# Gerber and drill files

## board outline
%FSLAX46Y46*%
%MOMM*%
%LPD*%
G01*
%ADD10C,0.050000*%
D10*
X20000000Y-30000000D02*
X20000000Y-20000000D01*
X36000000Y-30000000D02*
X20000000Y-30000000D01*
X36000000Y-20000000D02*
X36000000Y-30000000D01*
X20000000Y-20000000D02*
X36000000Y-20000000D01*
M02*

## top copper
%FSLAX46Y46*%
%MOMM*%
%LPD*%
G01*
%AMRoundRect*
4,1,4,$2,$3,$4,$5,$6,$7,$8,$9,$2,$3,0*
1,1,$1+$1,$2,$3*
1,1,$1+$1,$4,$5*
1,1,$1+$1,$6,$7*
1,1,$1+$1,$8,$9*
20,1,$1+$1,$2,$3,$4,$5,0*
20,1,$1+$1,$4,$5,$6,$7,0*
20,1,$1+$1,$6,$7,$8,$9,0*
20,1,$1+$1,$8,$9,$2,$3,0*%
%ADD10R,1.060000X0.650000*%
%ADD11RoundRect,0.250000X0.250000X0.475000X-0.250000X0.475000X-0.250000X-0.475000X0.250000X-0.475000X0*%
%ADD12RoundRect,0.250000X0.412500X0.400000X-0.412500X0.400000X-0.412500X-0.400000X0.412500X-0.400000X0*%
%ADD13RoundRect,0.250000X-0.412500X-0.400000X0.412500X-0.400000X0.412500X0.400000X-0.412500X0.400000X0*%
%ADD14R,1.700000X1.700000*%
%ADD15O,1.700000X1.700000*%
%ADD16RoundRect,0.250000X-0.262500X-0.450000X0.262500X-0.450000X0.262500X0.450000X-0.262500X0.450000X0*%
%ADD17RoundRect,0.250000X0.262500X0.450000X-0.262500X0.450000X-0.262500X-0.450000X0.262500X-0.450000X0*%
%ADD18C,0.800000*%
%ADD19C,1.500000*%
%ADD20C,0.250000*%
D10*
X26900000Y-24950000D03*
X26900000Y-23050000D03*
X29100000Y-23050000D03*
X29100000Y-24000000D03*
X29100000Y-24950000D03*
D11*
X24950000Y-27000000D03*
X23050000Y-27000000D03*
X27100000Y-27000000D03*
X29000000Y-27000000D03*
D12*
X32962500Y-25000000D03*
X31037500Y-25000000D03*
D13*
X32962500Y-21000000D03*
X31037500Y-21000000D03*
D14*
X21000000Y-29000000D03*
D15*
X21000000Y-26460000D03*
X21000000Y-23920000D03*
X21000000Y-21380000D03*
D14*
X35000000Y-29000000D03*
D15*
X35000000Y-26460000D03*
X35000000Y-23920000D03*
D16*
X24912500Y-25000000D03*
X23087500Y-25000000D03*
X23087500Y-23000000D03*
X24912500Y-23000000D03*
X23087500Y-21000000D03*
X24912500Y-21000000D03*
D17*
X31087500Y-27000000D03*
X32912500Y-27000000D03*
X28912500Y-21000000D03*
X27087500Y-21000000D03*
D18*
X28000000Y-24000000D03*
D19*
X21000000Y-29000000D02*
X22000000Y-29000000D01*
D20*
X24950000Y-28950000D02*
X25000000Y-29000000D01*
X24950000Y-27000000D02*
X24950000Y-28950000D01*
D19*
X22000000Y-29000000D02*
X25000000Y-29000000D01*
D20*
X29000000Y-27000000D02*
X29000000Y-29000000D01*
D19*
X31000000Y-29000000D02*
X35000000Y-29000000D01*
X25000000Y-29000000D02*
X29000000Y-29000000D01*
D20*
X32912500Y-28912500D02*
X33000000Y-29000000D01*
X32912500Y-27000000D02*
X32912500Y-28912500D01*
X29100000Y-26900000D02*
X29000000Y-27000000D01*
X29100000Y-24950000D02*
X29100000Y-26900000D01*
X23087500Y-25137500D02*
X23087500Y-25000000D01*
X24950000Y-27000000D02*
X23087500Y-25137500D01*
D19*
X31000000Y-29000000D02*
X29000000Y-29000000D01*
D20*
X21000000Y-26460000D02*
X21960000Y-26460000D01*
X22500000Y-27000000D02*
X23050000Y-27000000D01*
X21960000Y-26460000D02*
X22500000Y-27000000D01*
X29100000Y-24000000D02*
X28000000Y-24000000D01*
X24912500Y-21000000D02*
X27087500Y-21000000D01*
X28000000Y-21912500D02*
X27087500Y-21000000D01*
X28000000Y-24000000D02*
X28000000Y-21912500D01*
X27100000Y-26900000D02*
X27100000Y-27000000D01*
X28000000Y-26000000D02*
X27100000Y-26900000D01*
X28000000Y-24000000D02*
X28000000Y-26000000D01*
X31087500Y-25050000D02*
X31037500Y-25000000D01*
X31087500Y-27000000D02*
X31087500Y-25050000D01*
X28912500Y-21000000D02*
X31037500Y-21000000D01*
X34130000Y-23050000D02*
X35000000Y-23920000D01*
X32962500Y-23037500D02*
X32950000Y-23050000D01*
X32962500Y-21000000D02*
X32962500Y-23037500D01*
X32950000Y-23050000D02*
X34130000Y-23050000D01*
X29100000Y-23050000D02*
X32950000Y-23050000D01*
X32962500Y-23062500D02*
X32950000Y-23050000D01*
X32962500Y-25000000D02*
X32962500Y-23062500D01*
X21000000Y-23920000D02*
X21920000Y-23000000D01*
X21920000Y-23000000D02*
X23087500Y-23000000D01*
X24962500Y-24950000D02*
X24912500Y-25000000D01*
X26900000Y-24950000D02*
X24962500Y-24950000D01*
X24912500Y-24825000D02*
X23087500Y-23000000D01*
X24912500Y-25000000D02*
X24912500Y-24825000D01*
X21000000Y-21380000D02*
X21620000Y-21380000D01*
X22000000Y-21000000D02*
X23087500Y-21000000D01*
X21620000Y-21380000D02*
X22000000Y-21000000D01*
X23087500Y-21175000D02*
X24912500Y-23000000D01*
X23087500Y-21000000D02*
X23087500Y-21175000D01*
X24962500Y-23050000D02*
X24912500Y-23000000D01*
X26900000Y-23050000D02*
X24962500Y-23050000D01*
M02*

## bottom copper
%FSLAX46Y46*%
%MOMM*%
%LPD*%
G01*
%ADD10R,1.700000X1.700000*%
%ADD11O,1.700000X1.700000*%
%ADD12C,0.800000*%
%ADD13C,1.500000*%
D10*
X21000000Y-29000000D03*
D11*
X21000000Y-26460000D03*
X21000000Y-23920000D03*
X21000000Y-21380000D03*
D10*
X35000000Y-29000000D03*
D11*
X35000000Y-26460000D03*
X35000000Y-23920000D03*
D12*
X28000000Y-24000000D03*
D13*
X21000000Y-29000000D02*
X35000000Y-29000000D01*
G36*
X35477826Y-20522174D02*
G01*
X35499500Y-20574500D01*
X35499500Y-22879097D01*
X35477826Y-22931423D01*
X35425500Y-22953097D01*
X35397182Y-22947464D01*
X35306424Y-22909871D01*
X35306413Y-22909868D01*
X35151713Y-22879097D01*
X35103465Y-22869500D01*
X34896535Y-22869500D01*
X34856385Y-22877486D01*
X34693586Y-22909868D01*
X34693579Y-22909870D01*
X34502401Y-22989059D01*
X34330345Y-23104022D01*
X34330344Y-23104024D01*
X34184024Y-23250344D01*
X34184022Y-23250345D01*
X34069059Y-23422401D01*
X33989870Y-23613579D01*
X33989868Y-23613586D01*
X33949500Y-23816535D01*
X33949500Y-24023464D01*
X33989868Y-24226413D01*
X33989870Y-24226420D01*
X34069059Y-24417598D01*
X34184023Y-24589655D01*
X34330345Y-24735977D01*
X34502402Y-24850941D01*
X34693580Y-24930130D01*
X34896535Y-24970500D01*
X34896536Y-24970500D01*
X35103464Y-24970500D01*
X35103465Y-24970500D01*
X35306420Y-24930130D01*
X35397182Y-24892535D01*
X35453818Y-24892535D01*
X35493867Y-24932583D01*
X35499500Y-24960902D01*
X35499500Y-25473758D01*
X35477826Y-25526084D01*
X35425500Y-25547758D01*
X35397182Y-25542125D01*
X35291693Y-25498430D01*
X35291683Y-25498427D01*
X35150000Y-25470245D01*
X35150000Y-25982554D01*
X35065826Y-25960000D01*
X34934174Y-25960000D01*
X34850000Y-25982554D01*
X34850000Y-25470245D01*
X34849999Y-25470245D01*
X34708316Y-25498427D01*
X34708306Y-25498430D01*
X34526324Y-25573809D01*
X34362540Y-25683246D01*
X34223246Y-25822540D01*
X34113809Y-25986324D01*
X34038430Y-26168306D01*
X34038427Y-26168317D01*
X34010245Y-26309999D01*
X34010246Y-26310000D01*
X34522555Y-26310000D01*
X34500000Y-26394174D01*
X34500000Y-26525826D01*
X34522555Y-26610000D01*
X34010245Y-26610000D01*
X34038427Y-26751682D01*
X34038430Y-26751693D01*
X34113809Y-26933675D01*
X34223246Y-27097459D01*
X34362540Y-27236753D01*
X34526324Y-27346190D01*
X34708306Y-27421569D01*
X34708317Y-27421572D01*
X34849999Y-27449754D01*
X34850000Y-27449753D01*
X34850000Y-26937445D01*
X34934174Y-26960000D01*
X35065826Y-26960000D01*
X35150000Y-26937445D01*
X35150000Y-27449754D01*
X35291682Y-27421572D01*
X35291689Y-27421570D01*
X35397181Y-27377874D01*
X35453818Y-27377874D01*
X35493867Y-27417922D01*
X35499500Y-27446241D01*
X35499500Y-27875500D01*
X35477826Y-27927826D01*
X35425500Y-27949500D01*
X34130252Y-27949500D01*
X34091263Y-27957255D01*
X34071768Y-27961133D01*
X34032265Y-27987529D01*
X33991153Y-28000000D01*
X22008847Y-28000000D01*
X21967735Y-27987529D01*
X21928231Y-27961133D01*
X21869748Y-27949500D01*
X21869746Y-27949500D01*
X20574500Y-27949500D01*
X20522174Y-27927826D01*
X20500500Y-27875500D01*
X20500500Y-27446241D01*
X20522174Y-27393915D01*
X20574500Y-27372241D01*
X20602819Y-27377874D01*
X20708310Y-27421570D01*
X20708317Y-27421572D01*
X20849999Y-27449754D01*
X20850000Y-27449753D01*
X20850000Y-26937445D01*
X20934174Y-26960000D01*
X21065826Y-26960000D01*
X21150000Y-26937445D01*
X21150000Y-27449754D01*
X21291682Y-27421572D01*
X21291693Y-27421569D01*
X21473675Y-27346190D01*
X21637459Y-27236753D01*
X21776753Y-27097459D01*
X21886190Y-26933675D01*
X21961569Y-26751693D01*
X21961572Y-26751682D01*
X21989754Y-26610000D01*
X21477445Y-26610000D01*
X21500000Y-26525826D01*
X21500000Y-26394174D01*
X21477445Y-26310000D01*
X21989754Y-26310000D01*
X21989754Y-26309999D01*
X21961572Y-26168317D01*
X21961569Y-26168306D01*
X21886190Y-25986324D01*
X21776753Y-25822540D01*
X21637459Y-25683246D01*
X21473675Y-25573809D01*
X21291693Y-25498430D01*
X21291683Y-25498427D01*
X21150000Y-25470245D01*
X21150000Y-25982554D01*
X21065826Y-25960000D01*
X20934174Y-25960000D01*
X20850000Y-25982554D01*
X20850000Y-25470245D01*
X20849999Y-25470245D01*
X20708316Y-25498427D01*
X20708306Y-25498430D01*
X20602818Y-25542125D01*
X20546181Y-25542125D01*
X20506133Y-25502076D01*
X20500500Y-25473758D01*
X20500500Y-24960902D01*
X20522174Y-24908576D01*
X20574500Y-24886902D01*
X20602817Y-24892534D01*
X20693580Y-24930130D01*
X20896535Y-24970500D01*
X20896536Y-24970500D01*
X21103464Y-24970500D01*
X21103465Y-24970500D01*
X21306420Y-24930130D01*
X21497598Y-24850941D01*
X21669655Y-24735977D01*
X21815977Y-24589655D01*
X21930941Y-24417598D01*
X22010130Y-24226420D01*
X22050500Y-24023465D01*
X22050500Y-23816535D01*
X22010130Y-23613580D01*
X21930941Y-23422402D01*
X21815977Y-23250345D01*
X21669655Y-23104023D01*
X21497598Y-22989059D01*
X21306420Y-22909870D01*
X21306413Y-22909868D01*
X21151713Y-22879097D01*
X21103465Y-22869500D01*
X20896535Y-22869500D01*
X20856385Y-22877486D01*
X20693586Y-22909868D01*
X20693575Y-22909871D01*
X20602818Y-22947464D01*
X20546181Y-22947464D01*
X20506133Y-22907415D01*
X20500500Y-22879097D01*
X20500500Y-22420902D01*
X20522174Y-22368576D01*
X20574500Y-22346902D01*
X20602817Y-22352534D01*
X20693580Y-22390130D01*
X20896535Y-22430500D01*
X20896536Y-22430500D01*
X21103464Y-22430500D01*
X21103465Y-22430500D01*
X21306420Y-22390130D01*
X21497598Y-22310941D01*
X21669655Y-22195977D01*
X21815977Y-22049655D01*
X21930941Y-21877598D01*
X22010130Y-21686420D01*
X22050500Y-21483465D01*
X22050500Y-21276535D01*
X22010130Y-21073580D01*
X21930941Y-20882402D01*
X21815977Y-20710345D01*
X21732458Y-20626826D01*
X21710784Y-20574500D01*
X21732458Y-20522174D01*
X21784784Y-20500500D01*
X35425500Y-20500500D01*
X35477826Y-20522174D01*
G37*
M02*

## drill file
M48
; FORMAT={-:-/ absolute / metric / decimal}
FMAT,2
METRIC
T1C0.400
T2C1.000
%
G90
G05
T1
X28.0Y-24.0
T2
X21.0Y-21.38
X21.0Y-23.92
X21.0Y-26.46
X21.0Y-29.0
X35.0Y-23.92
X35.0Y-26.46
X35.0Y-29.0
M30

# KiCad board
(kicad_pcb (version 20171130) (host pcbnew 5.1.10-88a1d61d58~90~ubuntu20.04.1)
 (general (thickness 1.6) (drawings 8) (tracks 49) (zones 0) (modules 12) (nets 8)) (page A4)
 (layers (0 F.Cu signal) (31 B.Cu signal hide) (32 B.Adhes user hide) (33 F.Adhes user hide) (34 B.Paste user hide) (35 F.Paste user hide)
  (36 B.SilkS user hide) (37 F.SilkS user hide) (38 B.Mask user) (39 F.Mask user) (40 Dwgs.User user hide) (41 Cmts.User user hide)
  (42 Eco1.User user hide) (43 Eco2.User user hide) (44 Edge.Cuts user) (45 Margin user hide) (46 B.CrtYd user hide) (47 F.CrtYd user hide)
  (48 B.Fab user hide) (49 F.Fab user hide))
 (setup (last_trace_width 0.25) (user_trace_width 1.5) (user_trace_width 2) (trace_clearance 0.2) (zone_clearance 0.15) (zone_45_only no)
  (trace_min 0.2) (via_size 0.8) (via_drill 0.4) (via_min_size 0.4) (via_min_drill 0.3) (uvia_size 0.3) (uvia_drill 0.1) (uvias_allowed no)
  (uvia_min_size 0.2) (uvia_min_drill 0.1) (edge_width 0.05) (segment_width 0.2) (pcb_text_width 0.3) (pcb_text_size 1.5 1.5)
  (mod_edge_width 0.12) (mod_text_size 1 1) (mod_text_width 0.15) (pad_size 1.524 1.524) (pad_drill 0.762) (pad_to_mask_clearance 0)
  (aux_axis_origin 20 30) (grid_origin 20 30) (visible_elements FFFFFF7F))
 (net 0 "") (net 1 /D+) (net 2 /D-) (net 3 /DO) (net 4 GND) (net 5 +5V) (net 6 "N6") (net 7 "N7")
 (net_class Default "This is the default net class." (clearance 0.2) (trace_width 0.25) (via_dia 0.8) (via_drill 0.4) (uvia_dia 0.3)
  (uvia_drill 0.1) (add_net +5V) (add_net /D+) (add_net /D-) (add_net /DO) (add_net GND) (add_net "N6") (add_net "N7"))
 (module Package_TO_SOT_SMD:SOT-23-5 (layer F.Cu) (at 28 24 180)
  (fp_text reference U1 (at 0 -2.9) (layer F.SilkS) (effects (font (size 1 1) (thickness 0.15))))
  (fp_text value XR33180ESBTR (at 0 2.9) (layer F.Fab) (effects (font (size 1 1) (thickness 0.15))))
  (pad 5 smd rect (at 1.1 -0.95 180) (size 1.06 0.65) (layers F.Cu F.Paste F.Mask) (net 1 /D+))
  (pad 4 smd rect (at 1.1 0.95 180) (size 1.06 0.65) (layers F.Cu F.Paste F.Mask) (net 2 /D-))
  (pad 3 smd rect (at -1.1 0.95 180) (size 1.06 0.65) (layers F.Cu F.Paste F.Mask) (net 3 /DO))
  (pad 2 smd rect (at -1.1 0 180) (size 1.06 0.65) (layers F.Cu F.Paste F.Mask) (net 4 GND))
  (pad 1 smd rect (at -1.1 -0.95 180) (size 1.06 0.65) (layers F.Cu F.Paste F.Mask) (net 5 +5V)))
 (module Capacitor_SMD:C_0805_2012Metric (layer F.Cu) (at 24 27 180)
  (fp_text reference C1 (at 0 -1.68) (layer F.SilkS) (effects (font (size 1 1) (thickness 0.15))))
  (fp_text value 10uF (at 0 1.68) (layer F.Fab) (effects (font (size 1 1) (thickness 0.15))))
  (pad 1 smd roundrect (at -0.95 0 180) (size 1 1.45) (layers F.Cu F.Paste F.Mask) (roundrect_rratio 0.25) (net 5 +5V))
  (pad 2 smd roundrect (at 0.95 0 180) (size 1 1.45) (layers F.Cu F.Paste F.Mask) (roundrect_rratio 0.25) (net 4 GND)))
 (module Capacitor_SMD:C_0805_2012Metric (layer F.Cu) (at 28.05 27 180)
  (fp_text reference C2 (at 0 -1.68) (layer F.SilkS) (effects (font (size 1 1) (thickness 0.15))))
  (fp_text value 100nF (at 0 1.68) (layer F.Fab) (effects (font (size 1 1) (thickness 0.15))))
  (pad 2 smd roundrect (at 0.95 0 180) (size 1 1.45) (layers F.Cu F.Paste F.Mask) (roundrect_rratio 0.25) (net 4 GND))
  (pad 1 smd roundrect (at -0.95 0 180) (size 1 1.45) (layers F.Cu F.Paste F.Mask) (roundrect_rratio 0.25) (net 5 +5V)))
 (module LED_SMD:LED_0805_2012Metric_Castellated (layer F.Cu) (at 32 25 180)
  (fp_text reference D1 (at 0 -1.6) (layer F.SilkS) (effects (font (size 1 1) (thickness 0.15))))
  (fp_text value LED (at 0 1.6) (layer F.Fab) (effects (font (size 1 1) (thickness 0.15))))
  (pad 1 smd roundrect (at -0.9625 0 180) (size 1.325 1.3) (layers F.Cu F.Paste F.Mask) (roundrect_rratio 0.192308) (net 3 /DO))
  (pad 2 smd roundrect (at 0.9625 0 180) (size 1.325 1.3) (layers F.Cu F.Paste F.Mask) (roundrect_rratio 0.192308) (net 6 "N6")))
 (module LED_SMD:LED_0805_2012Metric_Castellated (layer F.Cu) (at 32 21)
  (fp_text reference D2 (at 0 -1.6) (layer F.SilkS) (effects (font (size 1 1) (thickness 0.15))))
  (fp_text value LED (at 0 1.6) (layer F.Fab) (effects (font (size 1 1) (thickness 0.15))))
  (pad 2 smd roundrect (at 0.9625 0) (size 1.325 1.3) (layers F.Cu F.Paste F.Mask) (roundrect_rratio 0.192308) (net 3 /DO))
  (pad 1 smd roundrect (at -0.9625 0) (size 1.325 1.3) (layers F.Cu F.Paste F.Mask) (roundrect_rratio 0.192308) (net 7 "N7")))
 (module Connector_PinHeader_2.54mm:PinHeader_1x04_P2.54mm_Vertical (layer F.Cu) (at 21 29 180)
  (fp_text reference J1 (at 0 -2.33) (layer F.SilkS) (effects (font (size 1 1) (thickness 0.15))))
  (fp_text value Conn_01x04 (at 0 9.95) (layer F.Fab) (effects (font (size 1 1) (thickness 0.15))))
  (pad 1 thru_hole rect (at 0 0 180) (size 1.7 1.7) (drill 1) (layers *.Cu *.Mask) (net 5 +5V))
  (pad 2 thru_hole oval (at 0 2.54 180) (size 1.7 1.7) (drill 1) (layers *.Cu *.Mask) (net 4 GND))
  (pad 3 thru_hole oval (at 0 5.08 180) (size 1.7 1.7) (drill 1) (layers *.Cu *.Mask) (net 1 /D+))
  (pad 4 thru_hole oval (at 0 7.62 180) (size 1.7 1.7) (drill 1) (layers *.Cu *.Mask) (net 2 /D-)))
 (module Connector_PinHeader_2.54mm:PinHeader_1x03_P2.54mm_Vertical (layer F.Cu) (at 35 29 180)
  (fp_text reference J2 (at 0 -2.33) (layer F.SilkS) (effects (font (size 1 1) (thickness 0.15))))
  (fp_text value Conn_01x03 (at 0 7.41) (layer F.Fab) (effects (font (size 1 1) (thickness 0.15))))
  (pad 1 thru_hole rect (at 0 0 180) (size 1.7 1.7) (drill 1) (layers *.Cu *.Mask) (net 5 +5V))
  (pad 2 thru_hole oval (at 0 2.54 180) (size 1.7 1.7) (drill 1) (layers *.Cu *.Mask) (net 4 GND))
  (pad 3 thru_hole oval (at 0 5.08 180) (size 1.7 1.7) (drill 1) (layers *.Cu *.Mask) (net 3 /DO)))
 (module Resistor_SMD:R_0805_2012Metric (layer F.Cu) (at 24 25)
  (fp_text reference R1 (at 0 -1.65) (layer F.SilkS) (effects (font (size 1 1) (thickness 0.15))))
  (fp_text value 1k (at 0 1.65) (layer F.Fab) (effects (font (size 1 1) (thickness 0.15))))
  (pad 2 smd roundrect (at 0.9125 0) (size 1.025 1.4) (layers F.Cu F.Paste F.Mask) (roundrect_rratio 0.243902) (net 1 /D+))
  (pad 1 smd roundrect (at -0.9125 0) (size 1.025 1.4) (layers F.Cu F.Paste F.Mask) (roundrect_rratio 0.243902) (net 5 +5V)))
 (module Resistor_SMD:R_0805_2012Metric (layer F.Cu) (at 24 23)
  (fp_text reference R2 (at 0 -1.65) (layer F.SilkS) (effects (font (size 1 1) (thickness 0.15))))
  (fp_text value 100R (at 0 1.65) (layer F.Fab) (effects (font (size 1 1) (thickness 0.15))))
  (pad 1 smd roundrect (at -0.9125 0) (size 1.025 1.4) (layers F.Cu F.Paste F.Mask) (roundrect_rratio 0.243902) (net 1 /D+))
  (pad 2 smd roundrect (at 0.9125 0) (size 1.025 1.4) (layers F.Cu F.Paste F.Mask) (roundrect_rratio 0.243902) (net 2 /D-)))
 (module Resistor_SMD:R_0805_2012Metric (layer F.Cu) (at 24 21)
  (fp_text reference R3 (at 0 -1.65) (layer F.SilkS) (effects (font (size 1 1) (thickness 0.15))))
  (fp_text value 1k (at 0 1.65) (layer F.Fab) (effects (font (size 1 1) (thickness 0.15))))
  (pad 1 smd roundrect (at -0.9125 0) (size 1.025 1.4) (layers F.Cu F.Paste F.Mask) (roundrect_rratio 0.243902) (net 2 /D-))
  (pad 2 smd roundrect (at 0.9125 0) (size 1.025 1.4) (layers F.Cu F.Paste F.Mask) (roundrect_rratio 0.243902) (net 4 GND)))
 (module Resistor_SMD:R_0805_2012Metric (layer F.Cu) (at 32 27 180)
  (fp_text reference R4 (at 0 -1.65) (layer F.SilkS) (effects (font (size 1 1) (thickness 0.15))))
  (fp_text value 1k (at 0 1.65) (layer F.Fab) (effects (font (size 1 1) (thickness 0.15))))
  (pad 2 smd roundrect (at 0.9125 0 180) (size 1.025 1.4) (layers F.Cu F.Paste F.Mask) (roundrect_rratio 0.243902) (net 6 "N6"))
  (pad 1 smd roundrect (at -0.9125 0 180) (size 1.025 1.4) (layers F.Cu F.Paste F.Mask) (roundrect_rratio 0.243902) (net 5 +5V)))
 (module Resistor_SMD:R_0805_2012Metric (layer F.Cu) (at 28 21 180)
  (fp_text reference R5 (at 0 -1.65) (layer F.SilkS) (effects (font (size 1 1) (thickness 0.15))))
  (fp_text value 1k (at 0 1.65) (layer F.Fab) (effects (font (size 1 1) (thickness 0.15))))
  (pad 1 smd roundrect (at -0.9125 0 180) (size 1.025 1.4) (layers F.Cu F.Paste F.Mask) (roundrect_rratio 0.243902) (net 7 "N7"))
  (pad 2 smd roundrect (at 0.9125 0 180) (size 1.025 1.4) (layers F.Cu F.Paste F.Mask) (roundrect_rratio 0.243902) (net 4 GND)))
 (gr_line (start 20 30) (end 20 20) (layer Edge.Cuts) (width 0.05))
 (gr_line (start 36 30) (end 20 30) (layer Edge.Cuts) (width 0.05))
 (gr_line (start 36 20) (end 36 30) (layer Edge.Cuts) (width 0.05))
 (gr_line (start 20 20) (end 36 20) (layer Edge.Cuts) (width 0.05))
 (segment (start 21 29) (end 35 29) (width 1.5) (layer B.Cu) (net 5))
 (segment (start 21 29) (end 22 29) (width 1.5) (layer F.Cu) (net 5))
 (segment (start 24.95 28.95) (end 25 29) (width 0.25) (layer F.Cu) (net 5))
 (segment (start 24.95 27) (end 24.95 28.95) (width 0.25) (layer F.Cu) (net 5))
 (segment (start 22 29) (end 25 29) (width 1.5) (layer F.Cu) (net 5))
 (segment (start 29 27) (end 29 29) (width 0.25) (layer F.Cu) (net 5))
 (segment (start 31 29) (end 35 29) (width 1.5) (layer F.Cu) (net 5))
 (segment (start 25 29) (end 29 29) (width 1.5) (layer F.Cu) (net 5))
 (segment (start 32.9125 28.9125) (end 33 29) (width 0.25) (layer F.Cu) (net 5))
 (segment (start 32.9125 27) (end 32.9125 28.9125) (width 0.25) (layer F.Cu) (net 5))
 (segment (start 29.1 26.9) (end 29 27) (width 0.25) (layer F.Cu) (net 5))
 (segment (start 29.1 24.95) (end 29.1 26.9) (width 0.25) (layer F.Cu) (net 5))
 (segment (start 23.0875 25.1375) (end 23.0875 25) (width 0.25) (layer F.Cu) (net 5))
 (segment (start 24.95 27) (end 23.0875 25.1375) (width 0.25) (layer F.Cu) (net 5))
 (segment (start 31 29) (end 29 29) (width 1.5) (layer F.Cu) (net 5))
 (via (at 28 24) (size 0.8) (drill 0.4) (layers F.Cu B.Cu) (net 4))
 (segment (start 21 26.46) (end 21.96 26.46) (width 0.25) (layer F.Cu) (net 4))
 (segment (start 22.5 27) (end 23.05 27) (width 0.25) (layer F.Cu) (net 4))
 (segment (start 21.96 26.46) (end 22.5 27) (width 0.25) (layer F.Cu) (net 4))
 (segment (start 29.1 24) (end 28 24) (width 0.25) (layer F.Cu) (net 4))
 (segment (start 24.9125 21) (end 27.0875 21) (width 0.25) (layer F.Cu) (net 4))
 (segment (start 28 21.9125) (end 27.0875 21) (width 0.25) (layer F.Cu) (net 4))
 (segment (start 28 24) (end 28 21.9125) (width 0.25) (layer F.Cu) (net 4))
 (segment (start 27.1 26.9) (end 27.1 27) (width 0.25) (layer F.Cu) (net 4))
 (segment (start 28 26) (end 27.1 26.9) (width 0.25) (layer F.Cu) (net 4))
 (segment (start 28 24) (end 28 26) (width 0.25) (layer F.Cu) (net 4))
 (segment (start 31.0875 25.05) (end 31.0375 25) (width 0.25) (layer F.Cu) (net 6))
 (segment (start 31.0875 27) (end 31.0875 25.05) (width 0.25) (layer F.Cu) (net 6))
 (segment (start 28.9125 21) (end 31.0375 21) (width 0.25) (layer F.Cu) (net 7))
 (segment (start 34.13 23.05) (end 35 23.92) (width 0.25) (layer F.Cu) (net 3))
 (segment (start 32.9625 23.0375) (end 32.95 23.05) (width 0.25) (layer F.Cu) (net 3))
 (segment (start 32.9625 21) (end 32.9625 23.0375) (width 0.25) (layer F.Cu) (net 3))
 (segment (start 32.95 23.05) (end 34.13 23.05) (width 0.25) (layer F.Cu) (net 3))
 (segment (start 29.1 23.05) (end 32.95 23.05) (width 0.25) (layer F.Cu) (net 3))
 (segment (start 32.9625 23.0625) (end 32.95 23.05) (width 0.25) (layer F.Cu) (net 3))
 (segment (start 32.9625 25) (end 32.9625 23.0625) (width 0.25) (layer F.Cu) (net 3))
 (segment (start 21 23.92) (end 21.92 23) (width 0.25) (layer F.Cu) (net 1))
 (segment (start 21.92 23) (end 23.0875 23) (width 0.25) (layer F.Cu) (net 1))
 (segment (start 24.9625 24.95) (end 24.9125 25) (width 0.25) (layer F.Cu) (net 1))
 (segment (start 26.9 24.95) (end 24.9625 24.95) (width 0.25) (layer F.Cu) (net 1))
 (segment (start 24.9125 24.825) (end 23.0875 23) (width 0.25) (layer F.Cu) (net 1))
 (segment (start 24.9125 25) (end 24.9125 24.825) (width 0.25) (layer F.Cu) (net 1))
 (segment (start 21 21.38) (end 21.62 21.38) (width 0.25) (layer F.Cu) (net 2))
 (segment (start 22 21) (end 23.0875 21) (width 0.25) (layer F.Cu) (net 2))
 (segment (start 21.62 21.38) (end 22 21) (width 0.25) (layer F.Cu) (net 2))
 (segment (start 23.0875 21.175) (end 24.9125 23) (width 0.25) (layer F.Cu) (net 2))
 (segment (start 23.0875 21) (end 23.0875 21.175) (width 0.25) (layer F.Cu) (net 2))
 (segment (start 24.9625 23.05) (end 24.9125 23) (width 0.25) (layer F.Cu) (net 2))
 (segment (start 26.9 23.05) (end 24.9625 23.05) (width 0.25) (layer F.Cu) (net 2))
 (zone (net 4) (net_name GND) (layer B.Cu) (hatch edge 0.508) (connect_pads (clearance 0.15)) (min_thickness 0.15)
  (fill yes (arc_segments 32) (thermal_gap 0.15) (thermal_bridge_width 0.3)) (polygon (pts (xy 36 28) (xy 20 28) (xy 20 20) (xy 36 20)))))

